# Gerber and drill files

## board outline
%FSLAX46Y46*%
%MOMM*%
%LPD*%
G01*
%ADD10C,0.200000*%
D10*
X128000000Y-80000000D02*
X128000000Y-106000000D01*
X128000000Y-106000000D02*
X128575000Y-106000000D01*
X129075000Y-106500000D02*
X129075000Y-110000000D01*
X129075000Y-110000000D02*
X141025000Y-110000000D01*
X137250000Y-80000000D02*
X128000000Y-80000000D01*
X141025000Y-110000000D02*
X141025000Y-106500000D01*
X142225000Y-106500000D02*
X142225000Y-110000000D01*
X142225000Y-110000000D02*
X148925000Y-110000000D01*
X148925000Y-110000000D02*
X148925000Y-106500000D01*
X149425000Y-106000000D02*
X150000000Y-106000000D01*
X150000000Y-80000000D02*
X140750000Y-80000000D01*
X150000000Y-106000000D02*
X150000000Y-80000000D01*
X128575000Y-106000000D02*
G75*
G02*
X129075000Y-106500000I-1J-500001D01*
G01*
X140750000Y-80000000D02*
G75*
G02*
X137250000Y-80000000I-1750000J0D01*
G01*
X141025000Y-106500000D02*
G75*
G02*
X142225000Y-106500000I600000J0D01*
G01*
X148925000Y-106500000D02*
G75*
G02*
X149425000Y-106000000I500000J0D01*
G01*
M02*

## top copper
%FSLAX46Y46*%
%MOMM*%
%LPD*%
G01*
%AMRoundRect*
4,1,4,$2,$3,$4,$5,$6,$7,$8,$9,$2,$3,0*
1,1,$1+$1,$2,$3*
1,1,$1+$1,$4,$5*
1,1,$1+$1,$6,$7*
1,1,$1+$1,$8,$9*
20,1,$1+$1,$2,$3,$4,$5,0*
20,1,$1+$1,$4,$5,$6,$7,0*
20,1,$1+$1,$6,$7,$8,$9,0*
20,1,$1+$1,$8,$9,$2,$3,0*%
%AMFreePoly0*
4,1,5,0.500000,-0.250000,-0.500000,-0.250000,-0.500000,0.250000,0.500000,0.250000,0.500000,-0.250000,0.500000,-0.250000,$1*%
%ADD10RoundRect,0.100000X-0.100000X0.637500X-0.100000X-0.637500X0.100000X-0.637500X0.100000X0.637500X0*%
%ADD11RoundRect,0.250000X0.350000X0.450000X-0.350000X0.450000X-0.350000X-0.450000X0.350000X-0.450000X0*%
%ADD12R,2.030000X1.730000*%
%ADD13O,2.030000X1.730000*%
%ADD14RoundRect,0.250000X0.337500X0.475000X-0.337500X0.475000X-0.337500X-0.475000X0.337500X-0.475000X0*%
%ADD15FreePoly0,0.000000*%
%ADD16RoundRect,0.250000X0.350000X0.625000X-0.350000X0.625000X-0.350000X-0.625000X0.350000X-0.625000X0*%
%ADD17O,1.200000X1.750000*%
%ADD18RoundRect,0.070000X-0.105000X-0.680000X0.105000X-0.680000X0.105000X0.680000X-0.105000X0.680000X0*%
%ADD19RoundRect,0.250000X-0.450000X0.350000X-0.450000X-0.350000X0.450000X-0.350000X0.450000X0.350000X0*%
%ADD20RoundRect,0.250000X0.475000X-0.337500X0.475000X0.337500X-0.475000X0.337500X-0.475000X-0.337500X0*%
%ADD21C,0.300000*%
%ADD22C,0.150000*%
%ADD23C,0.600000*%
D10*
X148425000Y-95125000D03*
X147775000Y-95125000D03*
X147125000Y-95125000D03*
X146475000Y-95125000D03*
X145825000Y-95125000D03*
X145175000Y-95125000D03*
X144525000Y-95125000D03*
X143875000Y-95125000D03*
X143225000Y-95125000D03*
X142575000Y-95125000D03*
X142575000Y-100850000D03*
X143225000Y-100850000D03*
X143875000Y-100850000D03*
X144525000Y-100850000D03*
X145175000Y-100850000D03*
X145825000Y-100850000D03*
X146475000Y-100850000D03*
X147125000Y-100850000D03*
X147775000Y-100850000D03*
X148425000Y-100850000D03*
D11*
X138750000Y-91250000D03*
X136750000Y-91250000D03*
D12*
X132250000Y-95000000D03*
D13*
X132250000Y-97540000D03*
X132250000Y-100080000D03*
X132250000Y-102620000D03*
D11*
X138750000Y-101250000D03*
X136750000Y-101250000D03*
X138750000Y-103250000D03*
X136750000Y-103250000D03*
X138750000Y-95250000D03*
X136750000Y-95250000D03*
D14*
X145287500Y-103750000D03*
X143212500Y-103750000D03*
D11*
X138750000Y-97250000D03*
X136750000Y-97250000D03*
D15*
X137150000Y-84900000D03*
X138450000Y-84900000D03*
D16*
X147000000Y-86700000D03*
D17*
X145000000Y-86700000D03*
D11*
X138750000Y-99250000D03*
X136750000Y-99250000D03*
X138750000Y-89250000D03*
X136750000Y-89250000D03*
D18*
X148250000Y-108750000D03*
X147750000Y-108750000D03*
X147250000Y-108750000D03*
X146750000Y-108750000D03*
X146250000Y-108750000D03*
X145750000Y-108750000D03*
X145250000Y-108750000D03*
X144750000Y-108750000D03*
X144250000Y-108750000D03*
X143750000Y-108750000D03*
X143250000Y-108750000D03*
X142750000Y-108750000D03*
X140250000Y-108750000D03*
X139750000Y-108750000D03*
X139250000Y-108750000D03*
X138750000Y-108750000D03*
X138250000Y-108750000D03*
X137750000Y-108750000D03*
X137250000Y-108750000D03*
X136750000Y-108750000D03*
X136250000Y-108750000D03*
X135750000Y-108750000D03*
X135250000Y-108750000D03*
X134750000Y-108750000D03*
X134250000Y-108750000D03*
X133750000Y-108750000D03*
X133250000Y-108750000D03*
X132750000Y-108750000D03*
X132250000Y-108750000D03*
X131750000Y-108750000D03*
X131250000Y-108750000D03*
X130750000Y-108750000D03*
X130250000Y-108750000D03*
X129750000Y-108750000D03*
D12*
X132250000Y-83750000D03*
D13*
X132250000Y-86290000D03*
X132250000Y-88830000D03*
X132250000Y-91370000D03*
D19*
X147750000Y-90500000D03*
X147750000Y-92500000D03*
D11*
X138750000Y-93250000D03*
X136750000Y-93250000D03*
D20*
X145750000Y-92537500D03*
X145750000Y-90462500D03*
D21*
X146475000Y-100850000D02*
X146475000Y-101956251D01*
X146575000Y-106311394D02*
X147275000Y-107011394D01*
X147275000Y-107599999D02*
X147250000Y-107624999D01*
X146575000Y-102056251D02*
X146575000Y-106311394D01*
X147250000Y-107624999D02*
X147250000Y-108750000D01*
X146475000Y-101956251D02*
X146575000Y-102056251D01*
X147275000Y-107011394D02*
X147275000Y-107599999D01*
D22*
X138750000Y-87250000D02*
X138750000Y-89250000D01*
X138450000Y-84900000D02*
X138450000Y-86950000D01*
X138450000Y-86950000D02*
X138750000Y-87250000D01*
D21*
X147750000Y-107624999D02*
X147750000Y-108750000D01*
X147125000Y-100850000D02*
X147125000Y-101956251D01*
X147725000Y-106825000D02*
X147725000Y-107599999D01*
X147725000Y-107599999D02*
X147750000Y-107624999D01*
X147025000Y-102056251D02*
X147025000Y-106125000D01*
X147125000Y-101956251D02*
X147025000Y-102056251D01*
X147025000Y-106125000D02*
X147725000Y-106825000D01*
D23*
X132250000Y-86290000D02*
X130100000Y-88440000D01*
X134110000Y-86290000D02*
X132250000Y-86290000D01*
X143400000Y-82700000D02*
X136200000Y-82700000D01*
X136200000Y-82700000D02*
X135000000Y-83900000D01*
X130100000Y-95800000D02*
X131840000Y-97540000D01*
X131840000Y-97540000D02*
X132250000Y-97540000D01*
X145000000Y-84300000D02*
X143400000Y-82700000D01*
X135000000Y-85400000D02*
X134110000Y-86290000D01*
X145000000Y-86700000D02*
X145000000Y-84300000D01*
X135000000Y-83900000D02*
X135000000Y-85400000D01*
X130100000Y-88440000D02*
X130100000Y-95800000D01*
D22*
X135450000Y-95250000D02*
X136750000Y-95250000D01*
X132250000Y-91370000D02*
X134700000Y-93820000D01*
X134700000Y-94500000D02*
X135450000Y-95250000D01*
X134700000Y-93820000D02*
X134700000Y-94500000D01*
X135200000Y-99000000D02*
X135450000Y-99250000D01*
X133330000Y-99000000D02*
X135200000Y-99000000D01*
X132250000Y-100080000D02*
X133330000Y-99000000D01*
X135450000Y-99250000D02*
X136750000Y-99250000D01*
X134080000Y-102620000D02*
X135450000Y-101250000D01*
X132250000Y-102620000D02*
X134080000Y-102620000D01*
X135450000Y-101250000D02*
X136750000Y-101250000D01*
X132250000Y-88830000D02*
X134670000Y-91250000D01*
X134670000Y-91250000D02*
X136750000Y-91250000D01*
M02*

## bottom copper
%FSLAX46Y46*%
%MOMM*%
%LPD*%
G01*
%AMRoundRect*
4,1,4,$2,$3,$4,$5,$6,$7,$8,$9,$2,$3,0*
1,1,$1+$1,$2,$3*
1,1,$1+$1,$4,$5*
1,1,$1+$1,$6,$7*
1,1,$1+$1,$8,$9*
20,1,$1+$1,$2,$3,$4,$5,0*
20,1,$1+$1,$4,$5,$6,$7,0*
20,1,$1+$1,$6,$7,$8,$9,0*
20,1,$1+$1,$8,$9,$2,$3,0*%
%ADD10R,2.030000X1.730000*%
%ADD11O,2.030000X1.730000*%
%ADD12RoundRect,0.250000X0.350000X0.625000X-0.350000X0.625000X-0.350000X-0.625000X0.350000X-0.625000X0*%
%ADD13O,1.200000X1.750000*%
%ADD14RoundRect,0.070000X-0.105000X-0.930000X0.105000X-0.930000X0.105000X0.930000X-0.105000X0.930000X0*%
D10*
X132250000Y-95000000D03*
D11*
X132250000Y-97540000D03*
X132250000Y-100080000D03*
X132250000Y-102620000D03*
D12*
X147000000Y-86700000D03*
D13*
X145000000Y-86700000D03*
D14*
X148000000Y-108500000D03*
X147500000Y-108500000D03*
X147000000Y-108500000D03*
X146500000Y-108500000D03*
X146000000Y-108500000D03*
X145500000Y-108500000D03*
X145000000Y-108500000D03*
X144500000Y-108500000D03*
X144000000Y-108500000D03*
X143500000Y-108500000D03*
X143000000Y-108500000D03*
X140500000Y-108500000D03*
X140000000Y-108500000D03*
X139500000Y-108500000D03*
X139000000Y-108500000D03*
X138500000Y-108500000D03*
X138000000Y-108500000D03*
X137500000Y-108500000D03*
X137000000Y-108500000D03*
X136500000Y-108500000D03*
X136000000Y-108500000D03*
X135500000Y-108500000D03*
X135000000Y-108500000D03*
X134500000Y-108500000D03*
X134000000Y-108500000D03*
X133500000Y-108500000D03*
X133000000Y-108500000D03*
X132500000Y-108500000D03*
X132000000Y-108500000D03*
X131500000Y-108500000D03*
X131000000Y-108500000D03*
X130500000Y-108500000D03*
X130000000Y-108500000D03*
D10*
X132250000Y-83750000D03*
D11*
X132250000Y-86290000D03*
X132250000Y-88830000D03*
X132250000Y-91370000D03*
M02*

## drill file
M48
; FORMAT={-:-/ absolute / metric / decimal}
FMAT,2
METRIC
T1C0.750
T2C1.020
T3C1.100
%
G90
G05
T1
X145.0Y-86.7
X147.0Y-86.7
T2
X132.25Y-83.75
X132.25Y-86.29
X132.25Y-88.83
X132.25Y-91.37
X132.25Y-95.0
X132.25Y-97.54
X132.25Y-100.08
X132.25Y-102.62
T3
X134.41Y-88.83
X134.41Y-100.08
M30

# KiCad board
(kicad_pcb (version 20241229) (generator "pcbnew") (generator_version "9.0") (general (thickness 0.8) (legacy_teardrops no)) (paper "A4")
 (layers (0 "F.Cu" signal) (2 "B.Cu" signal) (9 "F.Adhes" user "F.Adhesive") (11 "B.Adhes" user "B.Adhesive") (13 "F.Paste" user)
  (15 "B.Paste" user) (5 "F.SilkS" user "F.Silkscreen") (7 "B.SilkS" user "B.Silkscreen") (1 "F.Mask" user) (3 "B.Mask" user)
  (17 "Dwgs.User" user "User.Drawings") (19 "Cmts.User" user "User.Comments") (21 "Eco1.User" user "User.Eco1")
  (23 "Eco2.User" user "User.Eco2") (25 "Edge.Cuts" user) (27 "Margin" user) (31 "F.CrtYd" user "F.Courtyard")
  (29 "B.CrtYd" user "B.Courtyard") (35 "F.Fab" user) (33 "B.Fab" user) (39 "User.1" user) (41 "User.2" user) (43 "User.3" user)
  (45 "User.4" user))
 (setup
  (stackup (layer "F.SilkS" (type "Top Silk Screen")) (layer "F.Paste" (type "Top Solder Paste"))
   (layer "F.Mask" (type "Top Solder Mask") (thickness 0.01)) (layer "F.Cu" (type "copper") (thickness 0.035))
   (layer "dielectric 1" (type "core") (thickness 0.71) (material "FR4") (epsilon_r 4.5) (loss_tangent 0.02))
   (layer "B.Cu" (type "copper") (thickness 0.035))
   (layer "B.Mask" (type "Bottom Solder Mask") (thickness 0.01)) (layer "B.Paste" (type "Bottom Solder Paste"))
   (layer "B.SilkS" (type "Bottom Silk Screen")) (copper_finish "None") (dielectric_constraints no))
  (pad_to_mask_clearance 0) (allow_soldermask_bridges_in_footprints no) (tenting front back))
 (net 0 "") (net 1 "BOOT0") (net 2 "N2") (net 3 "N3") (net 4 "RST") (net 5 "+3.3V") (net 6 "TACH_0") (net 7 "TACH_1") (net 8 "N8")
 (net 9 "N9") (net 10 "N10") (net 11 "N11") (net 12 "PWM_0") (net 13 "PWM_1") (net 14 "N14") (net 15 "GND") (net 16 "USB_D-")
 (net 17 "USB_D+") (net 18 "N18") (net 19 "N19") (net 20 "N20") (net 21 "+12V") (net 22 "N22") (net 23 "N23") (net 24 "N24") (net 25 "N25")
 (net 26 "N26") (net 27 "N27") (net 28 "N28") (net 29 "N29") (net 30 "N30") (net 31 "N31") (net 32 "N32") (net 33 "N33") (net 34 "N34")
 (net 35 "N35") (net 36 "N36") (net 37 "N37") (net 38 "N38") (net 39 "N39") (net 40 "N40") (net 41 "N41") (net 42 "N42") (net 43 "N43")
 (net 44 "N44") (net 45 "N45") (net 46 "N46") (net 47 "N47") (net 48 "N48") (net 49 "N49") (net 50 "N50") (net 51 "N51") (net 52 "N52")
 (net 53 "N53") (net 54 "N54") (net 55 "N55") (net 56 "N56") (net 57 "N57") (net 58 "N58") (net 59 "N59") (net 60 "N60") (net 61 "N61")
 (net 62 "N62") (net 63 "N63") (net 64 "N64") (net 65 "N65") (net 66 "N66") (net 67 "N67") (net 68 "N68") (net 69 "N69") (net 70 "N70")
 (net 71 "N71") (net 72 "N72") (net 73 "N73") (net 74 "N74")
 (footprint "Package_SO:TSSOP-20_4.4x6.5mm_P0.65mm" (layer "F.Cu") (at 145.5 97.9875 -90)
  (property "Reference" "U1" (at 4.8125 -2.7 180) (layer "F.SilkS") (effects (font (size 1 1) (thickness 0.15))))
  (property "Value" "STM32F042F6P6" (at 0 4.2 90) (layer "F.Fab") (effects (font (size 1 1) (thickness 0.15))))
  (pad "1" smd roundrect (at -2.8625 -2.925 270) (size 1.475 0.4) (layers "F.Cu" "F.Mask" "F.Paste") (roundrect_rratio 0.25) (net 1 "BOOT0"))
  (pad "2" smd roundrect (at -2.8625 -2.275 270) (size 1.475 0.4) (layers "F.Cu" "F.Mask" "F.Paste") (roundrect_rratio 0.25) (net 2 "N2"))
  (pad "3" smd roundrect (at -2.8625 -1.625 270) (size 1.475 0.4) (layers "F.Cu" "F.Mask" "F.Paste") (roundrect_rratio 0.25) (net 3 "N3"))
  (pad "4" smd roundrect (at -2.8625 -0.975 270) (size 1.475 0.4) (layers "F.Cu" "F.Mask" "F.Paste") (roundrect_rratio 0.25) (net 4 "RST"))
  (pad "5" smd roundrect (at -2.8625 -0.325 270) (size 1.475 0.4) (layers "F.Cu" "F.Mask" "F.Paste") (roundrect_rratio 0.25) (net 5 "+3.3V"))
  (pad "6" smd roundrect (at -2.8625 0.325 270) (size 1.475 0.4) (layers "F.Cu" "F.Mask" "F.Paste") (roundrect_rratio 0.25) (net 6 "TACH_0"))
  (pad "7" smd roundrect (at -2.8625 0.975 270) (size 1.475 0.4) (layers "F.Cu" "F.Mask" "F.Paste") (roundrect_rratio 0.25) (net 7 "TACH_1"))
  (pad "8" smd roundrect (at -2.8625 1.625 270) (size 1.475 0.4) (layers "F.Cu" "F.Mask" "F.Paste") (roundrect_rratio 0.25) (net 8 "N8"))
  (pad "9" smd roundrect (at -2.8625 2.275 270) (size 1.475 0.4) (layers "F.Cu" "F.Mask" "F.Paste") (roundrect_rratio 0.25) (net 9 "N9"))
  (pad "10" smd roundrect (at -2.8625 2.925 270) (size 1.475 0.4) (layers "F.Cu" "F.Mask" "F.Paste") (roundrect_rratio 0.25) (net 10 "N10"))
  (pad "11" smd roundrect (at 2.8625 2.925 270) (size 1.475 0.4) (layers "F.Cu" "F.Mask" "F.Paste") (roundrect_rratio 0.25) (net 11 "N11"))
  (pad "12" smd roundrect (at 2.8625 2.275 270) (size 1.475 0.4) (layers "F.Cu" "F.Mask" "F.Paste") (roundrect_rratio 0.25) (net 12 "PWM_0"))
  (pad "13" smd roundrect (at 2.8625 1.625 270) (size 1.475 0.4) (layers "F.Cu" "F.Mask" "F.Paste") (roundrect_rratio 0.25) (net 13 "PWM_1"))
  (pad "14" smd roundrect (at 2.8625 0.975 270) (size 1.475 0.4) (layers "F.Cu" "F.Mask" "F.Paste") (roundrect_rratio 0.25) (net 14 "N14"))
  (pad "15" smd roundrect (at 2.8625 0.325 270) (size 1.475 0.4) (layers "F.Cu" "F.Mask" "F.Paste") (roundrect_rratio 0.25) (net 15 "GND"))
  (pad "16" smd roundrect (at 2.8625 -0.325 270) (size 1.475 0.4) (layers "F.Cu" "F.Mask" "F.Paste") (roundrect_rratio 0.25) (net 5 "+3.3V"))
  (pad "17" smd roundrect (at 2.8625 -0.975 270) (size 1.475 0.4) (layers "F.Cu" "F.Mask" "F.Paste") (roundrect_rratio 0.25)
   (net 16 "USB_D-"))
  (pad "18" smd roundrect (at 2.8625 -1.625 270) (size 1.475 0.4) (layers "F.Cu" "F.Mask" "F.Paste") (roundrect_rratio 0.25)
   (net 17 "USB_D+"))
  (pad "19" smd roundrect (at 2.8625 -2.275 270) (size 1.475 0.4) (layers "F.Cu" "F.Mask" "F.Paste") (roundrect_rratio 0.25) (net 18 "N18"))
  (pad "20" smd roundrect (at 2.8625 -2.925 270) (size 1.475 0.4) (layers "F.Cu" "F.Mask" "F.Paste") (roundrect_rratio 0.25) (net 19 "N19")))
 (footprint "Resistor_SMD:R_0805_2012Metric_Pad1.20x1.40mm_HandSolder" (layer "F.Cu") (at 137.75 91.25 180)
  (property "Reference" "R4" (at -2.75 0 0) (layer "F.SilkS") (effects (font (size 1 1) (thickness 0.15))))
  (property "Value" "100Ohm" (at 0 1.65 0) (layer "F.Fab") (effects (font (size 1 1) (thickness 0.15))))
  (pad "1" smd roundrect (at -1 0 180) (size 1.2 1.4) (layers "F.Cu" "F.Mask" "F.Paste") (roundrect_rratio 0.208333) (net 6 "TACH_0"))
  (pad "2" smd roundrect (at 1 0 180) (size 1.2 1.4) (layers "F.Cu" "F.Mask" "F.Paste") (roundrect_rratio 0.208333) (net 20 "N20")))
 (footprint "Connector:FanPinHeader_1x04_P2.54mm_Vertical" (layer "F.Cu") (at 132.25 95 -90)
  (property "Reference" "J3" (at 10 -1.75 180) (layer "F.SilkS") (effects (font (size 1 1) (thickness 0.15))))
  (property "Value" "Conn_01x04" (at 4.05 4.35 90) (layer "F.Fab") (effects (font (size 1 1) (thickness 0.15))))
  (pad "" np_thru_hole circle (at 5.08 -2.16) (size 1.1 1.1) (drill 1.1) (layers "*.Cu" "*.Mask"))
  (pad "1" thru_hole rect (at 0 0) (size 2.03 1.73) (drill 1.02) (layers "*.Cu" "*.Mask") (remove_unused_layers no) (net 15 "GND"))
  (pad "2" thru_hole oval (at 2.54 0) (size 2.03 1.73) (drill 1.02) (layers "*.Cu" "*.Mask") (remove_unused_layers no) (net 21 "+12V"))
  (pad "3" thru_hole oval (at 5.08 0) (size 2.03 1.73) (drill 1.02) (layers "*.Cu" "*.Mask") (remove_unused_layers no) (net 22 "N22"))
  (pad "4" thru_hole oval (at 7.62 0) (size 2.03 1.73) (drill 1.02) (layers "*.Cu" "*.Mask") (remove_unused_layers no) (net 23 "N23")))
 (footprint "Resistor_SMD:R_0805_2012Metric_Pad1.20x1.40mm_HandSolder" (layer "F.Cu") (at 137.75 101.25 180)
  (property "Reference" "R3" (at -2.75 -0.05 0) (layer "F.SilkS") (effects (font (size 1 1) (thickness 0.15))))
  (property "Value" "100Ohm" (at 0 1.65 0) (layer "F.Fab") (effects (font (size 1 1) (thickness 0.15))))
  (pad "1" smd roundrect (at -1 0 180) (size 1.2 1.4) (layers "F.Cu" "F.Mask" "F.Paste") (roundrect_rratio 0.208333) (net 13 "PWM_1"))
  (pad "2" smd roundrect (at 1 0 180) (size 1.2 1.4) (layers "F.Cu" "F.Mask" "F.Paste") (roundrect_rratio 0.208333) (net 23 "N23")))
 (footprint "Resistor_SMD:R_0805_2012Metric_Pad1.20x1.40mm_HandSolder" (layer "F.Cu") (at 137.75 103.25 180)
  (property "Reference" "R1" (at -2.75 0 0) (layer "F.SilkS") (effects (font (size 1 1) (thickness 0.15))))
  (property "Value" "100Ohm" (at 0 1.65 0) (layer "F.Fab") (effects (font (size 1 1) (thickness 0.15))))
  (pad "1" smd roundrect (at -1 0 180) (size 1.2 1.4) (layers "F.Cu" "F.Mask" "F.Paste") (roundrect_rratio 0.208333) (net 4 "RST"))
  (pad "2" smd roundrect (at 1 0 180) (size 1.2 1.4) (layers "F.Cu" "F.Mask" "F.Paste") (roundrect_rratio 0.208333) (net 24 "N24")))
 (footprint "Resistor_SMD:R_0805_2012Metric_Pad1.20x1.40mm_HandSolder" (layer "F.Cu") (at 137.75 95.25 180)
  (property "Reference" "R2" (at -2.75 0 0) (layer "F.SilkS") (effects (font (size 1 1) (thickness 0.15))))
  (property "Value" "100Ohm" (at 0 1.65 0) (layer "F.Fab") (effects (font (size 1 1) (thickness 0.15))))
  (pad "1" smd roundrect (at -1 0 180) (size 1.2 1.4) (layers "F.Cu" "F.Mask" "F.Paste") (roundrect_rratio 0.208333) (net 12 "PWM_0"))
  (pad "2" smd roundrect (at 1 0 180) (size 1.2 1.4) (layers "F.Cu" "F.Mask" "F.Paste") (roundrect_rratio 0.208333) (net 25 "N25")))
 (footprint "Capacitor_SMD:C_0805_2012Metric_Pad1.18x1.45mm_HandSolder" (layer "F.Cu") (at 144.25 103.75 180)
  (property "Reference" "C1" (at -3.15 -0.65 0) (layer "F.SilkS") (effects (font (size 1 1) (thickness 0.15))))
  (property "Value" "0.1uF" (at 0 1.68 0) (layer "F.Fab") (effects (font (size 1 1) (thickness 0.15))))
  (pad "1" smd roundrect (at -1.0375 0 180) (size 1.175 1.45) (layers "F.Cu" "F.Mask" "F.Paste") (roundrect_rratio 0.212766) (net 5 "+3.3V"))
  (pad "2" smd roundrect (at 1.0375 0 180) (size 1.175 1.45) (layers "F.Cu" "F.Mask" "F.Paste") (roundrect_rratio 0.212766) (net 15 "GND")))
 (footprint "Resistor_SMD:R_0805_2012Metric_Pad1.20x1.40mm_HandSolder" (layer "F.Cu") (at 137.75 97.25 180)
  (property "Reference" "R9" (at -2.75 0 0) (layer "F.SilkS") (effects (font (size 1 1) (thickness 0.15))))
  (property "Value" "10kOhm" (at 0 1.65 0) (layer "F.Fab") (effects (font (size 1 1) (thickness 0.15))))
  (pad "1" smd roundrect (at -1 0 180) (size 1.2 1.4) (layers "F.Cu" "F.Mask" "F.Paste") (roundrect_rratio 0.208333) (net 5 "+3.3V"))
  (pad "2" smd roundrect (at 1 0 180) (size 1.2 1.4) (layers "F.Cu" "F.Mask" "F.Paste") (roundrect_rratio 0.208333) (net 7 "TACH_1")))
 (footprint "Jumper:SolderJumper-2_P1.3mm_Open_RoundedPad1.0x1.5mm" (layer "F.Cu") (at 137.8 84.9)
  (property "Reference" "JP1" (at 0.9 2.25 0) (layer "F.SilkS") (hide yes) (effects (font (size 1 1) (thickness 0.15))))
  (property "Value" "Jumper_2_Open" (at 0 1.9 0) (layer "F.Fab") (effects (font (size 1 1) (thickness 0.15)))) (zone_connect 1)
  (pad "1" smd custom (at -0.65 0) (size 1 0.5) (layers "F.Cu" "F.Mask") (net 5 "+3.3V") (zone_connect 2) (thermal_bridge_angle 45)
   (options (clearance outline) (anchor rect)) (primitives))
  (pad "2" smd custom (at 0.65 0) (size 1 0.5) (layers "F.Cu" "F.Mask") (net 1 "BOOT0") (zone_connect 2) (thermal_bridge_angle 45)
   (options (clearance outline) (anchor rect)) (primitives)))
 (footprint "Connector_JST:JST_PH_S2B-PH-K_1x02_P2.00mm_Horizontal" (layer "F.Cu") (at 147 86.7 180)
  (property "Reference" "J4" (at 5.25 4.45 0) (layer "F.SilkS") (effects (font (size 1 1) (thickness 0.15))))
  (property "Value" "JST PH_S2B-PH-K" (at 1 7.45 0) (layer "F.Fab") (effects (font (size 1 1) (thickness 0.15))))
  (pad "1" thru_hole roundrect (at 0 0 180) (size 1.2 1.75) (drill 0.75) (layers "*.Cu" "*.Mask") (remove_unused_layers no)
   (roundrect_rratio 0.208333) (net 15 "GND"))
  (pad "2" thru_hole oval (at 2 0 180) (size 1.2 1.75) (drill 0.75) (layers "*.Cu" "*.Mask") (remove_unused_layers no) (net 21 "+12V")))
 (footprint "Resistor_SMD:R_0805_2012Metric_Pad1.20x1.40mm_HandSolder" (layer "F.Cu") (at 137.75 99.25 180)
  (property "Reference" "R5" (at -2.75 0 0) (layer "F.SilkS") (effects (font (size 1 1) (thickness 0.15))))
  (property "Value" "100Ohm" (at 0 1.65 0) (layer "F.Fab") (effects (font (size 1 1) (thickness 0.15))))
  (pad "1" smd roundrect (at -1 0 180) (size 1.2 1.4) (layers "F.Cu" "F.Mask" "F.Paste") (roundrect_rratio 0.208333) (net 7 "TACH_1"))
  (pad "2" smd roundrect (at 1 0 180) (size 1.2 1.4) (layers "F.Cu" "F.Mask" "F.Paste") (roundrect_rratio 0.208333) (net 22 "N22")))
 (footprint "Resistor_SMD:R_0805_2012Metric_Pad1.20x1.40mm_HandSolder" (layer "F.Cu") (at 137.75 89.25 180)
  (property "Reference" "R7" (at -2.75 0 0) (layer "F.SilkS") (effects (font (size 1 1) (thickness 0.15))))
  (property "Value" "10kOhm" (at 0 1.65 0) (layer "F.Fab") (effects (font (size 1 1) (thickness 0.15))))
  (pad "1" smd roundrect (at -1 0 180) (size 1.2 1.4) (layers "F.Cu" "F.Mask" "F.Paste") (roundrect_rratio 0.208333) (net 1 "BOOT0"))
  (pad "2" smd roundrect (at 1 0 180) (size 1.2 1.4) (layers "F.Cu" "F.Mask" "F.Paste") (roundrect_rratio 0.208333) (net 15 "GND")))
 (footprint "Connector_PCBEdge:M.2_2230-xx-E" (layer "F.Cu") (at 139 106)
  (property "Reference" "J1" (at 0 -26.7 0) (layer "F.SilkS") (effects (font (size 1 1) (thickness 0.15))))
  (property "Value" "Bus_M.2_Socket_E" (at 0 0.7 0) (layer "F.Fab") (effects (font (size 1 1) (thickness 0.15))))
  (fp_line (start -11 -26) (end -11 0) (stroke (width 0.2) (type solid)) (layer "Edge.Cuts"))
  (fp_line (start -11 0) (end -10.425 0) (stroke (width 0.2) (type solid)) (layer "Edge.Cuts"))
  (fp_line (start -9.925 0.5) (end -9.925 4) (stroke (width 0.2) (type solid)) (layer "Edge.Cuts"))
  (fp_line (start -9.925 4) (end 2.025 4) (stroke (width 0.2) (type solid)) (layer "Edge.Cuts"))
  (fp_line (start -1.75 -26) (end -11 -26) (stroke (width 0.2) (type solid)) (layer "Edge.Cuts"))
  (fp_line (start 2.025 4) (end 2.025 0.5) (stroke (width 0.2) (type solid)) (layer "Edge.Cuts"))
  (fp_line (start 3.225 0.5) (end 3.225 4) (stroke (width 0.2) (type solid)) (layer "Edge.Cuts"))
  (fp_line (start 3.225 4) (end 9.925 4) (stroke (width 0.2) (type solid)) (layer "Edge.Cuts"))
  (fp_line (start 9.925 4) (end 9.925 0.5) (stroke (width 0.2) (type solid)) (layer "Edge.Cuts"))
  (fp_line (start 10.425 0) (end 11 0) (stroke (width 0.2) (type solid)) (layer "Edge.Cuts"))
  (fp_line (start 11 -26) (end 1.75 -26) (stroke (width 0.2) (type solid)) (layer "Edge.Cuts"))
  (fp_line (start 11 0) (end 11 -26) (stroke (width 0.2) (type solid)) (layer "Edge.Cuts"))
  (fp_arc (start -10.425 0) (mid -10.071447 0.146447) (end -9.925 0.5) (stroke (width 0.2) (type solid)) (layer "Edge.Cuts"))
  (fp_arc (start 1.75 -26) (mid 0 -24.25) (end -1.75 -26) (stroke (width 0.2) (type solid)) (layer "Edge.Cuts"))
  (fp_arc (start 2.025 0.5) (mid 2.625 -0.1) (end 3.225 0.5) (stroke (width 0.2) (type solid)) (layer "Edge.Cuts"))
  (fp_arc (start 9.925 0.5) (mid 10.071447 0.146447) (end 10.425 0) (stroke (width 0.2) (type solid)) (layer "Edge.Cuts"))
  (pad "1" connect roundrect (at 9.25 2.75) (size 0.35 1.5) (layers "F.Cu" "F.Mask") (roundrect_rratio 0.2) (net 15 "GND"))
  (pad "2" connect roundrect (at 9 2.5) (size 0.35 2) (layers "B.Cu" "B.Mask") (roundrect_rratio 0.2) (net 5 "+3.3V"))
  (pad "3" connect roundrect (at 8.75 2.75) (size 0.35 1.5) (layers "F.Cu" "F.Mask") (roundrect_rratio 0.2) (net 17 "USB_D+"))
  (pad "4" connect roundrect (at 8.5 2.5) (size 0.35 2) (layers "B.Cu" "B.Mask") (roundrect_rratio 0.2) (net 5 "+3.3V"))
  (pad "5" connect roundrect (at 8.25 2.75) (size 0.35 1.5) (layers "F.Cu" "F.Mask") (roundrect_rratio 0.2) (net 16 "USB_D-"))
  (pad "6" connect roundrect (at 8 2.5) (size 0.35 2) (layers "B.Cu" "B.Mask") (roundrect_rratio 0.2) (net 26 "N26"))
  (pad "7" connect roundrect (at 7.75 2.75) (size 0.35 1.5) (layers "F.Cu" "F.Mask") (roundrect_rratio 0.2) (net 15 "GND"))
  (pad "8" connect roundrect (at 7.5 2.5) (size 0.35 2) (layers "B.Cu" "B.Mask") (roundrect_rratio 0.2) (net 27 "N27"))
  (pad "9" connect roundrect (at 7.25 2.75) (size 0.35 1.5) (layers "F.Cu" "F.Mask") (roundrect_rratio 0.2) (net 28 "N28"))
  (pad "10" connect roundrect (at 7 2.5) (size 0.35 2) (layers "B.Cu" "B.Mask") (roundrect_rratio 0.2) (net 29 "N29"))
  (pad "11" connect roundrect (at 6.75 2.75) (size 0.35 1.5) (layers "F.Cu" "F.Mask") (roundrect_rratio 0.2) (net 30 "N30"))
  (pad "12" connect roundrect (at 6.5 2.5) (size 0.35 2) (layers "B.Cu" "B.Mask") (roundrect_rratio 0.2) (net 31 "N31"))
  (pad "13" connect roundrect (at 6.25 2.75) (size 0.35 1.5) (layers "F.Cu" "F.Mask") (roundrect_rratio 0.2) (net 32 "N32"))
  (pad "14" connect roundrect (at 6 2.5) (size 0.35 2) (layers "B.Cu" "B.Mask") (roundrect_rratio 0.2) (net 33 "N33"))
  (pad "15" connect roundrect (at 5.75 2.75) (size 0.35 1.5) (layers "F.Cu" "F.Mask") (roundrect_rratio 0.2) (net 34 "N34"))
  (pad "16" connect roundrect (at 5.5 2.5) (size 0.35 2) (layers "B.Cu" "B.Mask") (roundrect_rratio 0.2) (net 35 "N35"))
  (pad "17" connect roundrect (at 5.25 2.75) (size 0.35 1.5) (layers "F.Cu" "F.Mask") (roundrect_rratio 0.2) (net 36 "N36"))
  (pad "18" connect roundrect (at 5 2.5) (size 0.35 2) (layers "B.Cu" "B.Mask") (roundrect_rratio 0.2) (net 15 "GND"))
  (pad "19" connect roundrect (at 4.75 2.75) (size 0.35 1.5) (layers "F.Cu" "F.Mask") (roundrect_rratio 0.2) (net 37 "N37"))
  (pad "20" connect roundrect (at 4.5 2.5) (size 0.35 2) (layers "B.Cu" "B.Mask") (roundrect_rratio 0.2) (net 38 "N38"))
  (pad "21" connect roundrect (at 4.25 2.75) (size 0.35 1.5) (layers "F.Cu" "F.Mask") (roundrect_rratio 0.2) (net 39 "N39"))
  (pad "22" connect roundrect (at 4 2.5) (size 0.35 2) (layers "B.Cu" "B.Mask") (roundrect_rratio 0.2) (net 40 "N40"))
  (pad "23" connect roundrect (at 3.75 2.75) (size 0.35 1.5) (layers "F.Cu" "F.Mask") (roundrect_rratio 0.2) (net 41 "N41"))
  (pad "32" connect roundrect (at 1.5 2.5) (size 0.35 2) (layers "B.Cu" "B.Mask") (roundrect_rratio 0.2) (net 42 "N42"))
  (pad "33" connect roundrect (at 1.25 2.75) (size 0.35 1.5) (layers "F.Cu" "F.Mask") (roundrect_rratio 0.2) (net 15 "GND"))
  (pad "34" connect roundrect (at 1 2.5) (size 0.35 2) (layers "B.Cu" "B.Mask") (roundrect_rratio 0.2) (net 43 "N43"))
  (pad "35" connect roundrect (at 0.75 2.75) (size 0.35 1.5) (layers "F.Cu" "F.Mask") (roundrect_rratio 0.2) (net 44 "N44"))
  (pad "36" connect roundrect (at 0.5 2.5) (size 0.35 2) (layers "B.Cu" "B.Mask") (roundrect_rratio 0.2) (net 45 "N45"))
  (pad "37" connect roundrect (at 0.25 2.75) (size 0.35 1.5) (layers "F.Cu" "F.Mask") (roundrect_rratio 0.2) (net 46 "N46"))
  (pad "38" connect roundrect (at 0 2.5) (size 0.35 2) (layers "B.Cu" "B.Mask") (roundrect_rratio 0.2) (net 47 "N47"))
  (pad "39" connect roundrect (at -0.25 2.75) (size 0.35 1.5) (layers "F.Cu" "F.Mask") (roundrect_rratio 0.2) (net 15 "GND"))
  (pad "40" connect roundrect (at -0.5 2.5) (size 0.35 2) (layers "B.Cu" "B.Mask") (roundrect_rratio 0.2) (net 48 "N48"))
  (pad "41" connect roundrect (at -0.75 2.75) (size 0.35 1.5) (layers "F.Cu" "F.Mask") (roundrect_rratio 0.2) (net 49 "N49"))
  (pad "42" connect roundrect (at -1 2.5) (size 0.35 2) (layers "B.Cu" "B.Mask") (roundrect_rratio 0.2) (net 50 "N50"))
  (pad "43" connect roundrect (at -1.25 2.75) (size 0.35 1.5) (layers "F.Cu" "F.Mask") (roundrect_rratio 0.2) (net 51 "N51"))
  (pad "44" connect roundrect (at -1.5 2.5) (size 0.35 2) (layers "B.Cu" "B.Mask") (roundrect_rratio 0.2) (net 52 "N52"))
  (pad "45" connect roundrect (at -1.75 2.75) (size 0.35 1.5) (layers "F.Cu" "F.Mask") (roundrect_rratio 0.2) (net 15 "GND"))
  (pad "46" connect roundrect (at -2 2.5) (size 0.35 2) (layers "B.Cu" "B.Mask") (roundrect_rratio 0.2) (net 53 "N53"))
  (pad "47" connect roundrect (at -2.25 2.75) (size 0.35 1.5) (layers "F.Cu" "F.Mask") (roundrect_rratio 0.2) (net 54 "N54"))
  (pad "48" connect roundrect (at -2.5 2.5) (size 0.35 2) (layers "B.Cu" "B.Mask") (roundrect_rratio 0.2) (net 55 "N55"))
  (pad "49" connect roundrect (at -2.75 2.75) (size 0.35 1.5) (layers "F.Cu" "F.Mask") (roundrect_rratio 0.2) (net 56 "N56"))
  (pad "50" connect roundrect (at -3 2.5) (size 0.35 2) (layers "B.Cu" "B.Mask") (roundrect_rratio 0.2) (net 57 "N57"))
  (pad "51" connect roundrect (at -3.25 2.75) (size 0.35 1.5) (layers "F.Cu" "F.Mask") (roundrect_rratio 0.2) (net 15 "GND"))
  (pad "52" connect roundrect (at -3.5 2.5) (size 0.35 2) (layers "B.Cu" "B.Mask") (roundrect_rratio 0.2) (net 24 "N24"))
  (pad "53" connect roundrect (at -3.75 2.75) (size 0.35 1.5) (layers "F.Cu" "F.Mask") (roundrect_rratio 0.2) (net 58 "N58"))
  (pad "54" connect roundrect (at -4 2.5) (size 0.35 2) (layers "B.Cu" "B.Mask") (roundrect_rratio 0.2) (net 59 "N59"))
  (pad "55" connect roundrect (at -4.25 2.75) (size 0.35 1.5) (layers "F.Cu" "F.Mask") (roundrect_rratio 0.2) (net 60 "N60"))
  (pad "56" connect roundrect (at -4.5 2.5) (size 0.35 2) (layers "B.Cu" "B.Mask") (roundrect_rratio 0.2) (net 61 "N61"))
  (pad "57" connect roundrect (at -4.75 2.75) (size 0.35 1.5) (layers "F.Cu" "F.Mask") (roundrect_rratio 0.2) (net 15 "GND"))
  (pad "58" connect roundrect (at -5 2.5) (size 0.35 2) (layers "B.Cu" "B.Mask") (roundrect_rratio 0.2) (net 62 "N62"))
  (pad "59" connect roundrect (at -5.25 2.75) (size 0.35 1.5) (layers "F.Cu" "F.Mask") (roundrect_rratio 0.2) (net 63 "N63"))
  (pad "60" connect roundrect (at -5.5 2.5) (size 0.35 2) (layers "B.Cu" "B.Mask") (roundrect_rratio 0.2) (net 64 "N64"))
  (pad "61" connect roundrect (at -5.75 2.75) (size 0.35 1.5) (layers "F.Cu" "F.Mask") (roundrect_rratio 0.2) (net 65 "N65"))
  (pad "62" connect roundrect (at -6 2.5) (size 0.35 2) (layers "B.Cu" "B.Mask") (roundrect_rratio 0.2) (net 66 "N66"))
  (pad "63" connect roundrect (at -6.25 2.75) (size 0.35 1.5) (layers "F.Cu" "F.Mask") (roundrect_rratio 0.2) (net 15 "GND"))
  (pad "64" connect roundrect (at -6.5 2.5) (size 0.35 2) (layers "B.Cu" "B.Mask") (roundrect_rratio 0.2) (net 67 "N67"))
  (pad "65" connect roundrect (at -6.75 2.75) (size 0.35 1.5) (layers "F.Cu" "F.Mask") (roundrect_rratio 0.2) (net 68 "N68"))
  (pad "66" connect roundrect (at -7 2.5) (size 0.35 2) (layers "B.Cu" "B.Mask") (roundrect_rratio 0.2) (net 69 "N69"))
  (pad "67" connect roundrect (at -7.25 2.75) (size 0.35 1.5) (layers "F.Cu" "F.Mask") (roundrect_rratio 0.2) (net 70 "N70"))
  (pad "68" connect roundrect (at -7.5 2.5) (size 0.35 2) (layers "B.Cu" "B.Mask") (roundrect_rratio 0.2) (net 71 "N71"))
  (pad "69" connect roundrect (at -7.75 2.75) (size 0.35 1.5) (layers "F.Cu" "F.Mask") (roundrect_rratio 0.2) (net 15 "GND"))
  (pad "70" connect roundrect (at -8 2.5) (size 0.35 2) (layers "B.Cu" "B.Mask") (roundrect_rratio 0.2) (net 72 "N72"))
  (pad "71" connect roundrect (at -8.25 2.75) (size 0.35 1.5) (layers "F.Cu" "F.Mask") (roundrect_rratio 0.2) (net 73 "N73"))
  (pad "72" connect roundrect (at -8.5 2.5) (size 0.35 2) (layers "B.Cu" "B.Mask") (roundrect_rratio 0.2) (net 5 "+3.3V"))
  (pad "73" connect roundrect (at -8.75 2.75) (size 0.35 1.5) (layers "F.Cu" "F.Mask") (roundrect_rratio 0.2) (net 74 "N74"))
  (pad "74" connect roundrect (at -9 2.5) (size 0.35 2) (layers "B.Cu" "B.Mask") (roundrect_rratio 0.2) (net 5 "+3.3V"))
  (pad "75" connect roundrect (at -9.25 2.75) (size 0.35 1.5) (layers "F.Cu" "F.Mask") (roundrect_rratio 0.2) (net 15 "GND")))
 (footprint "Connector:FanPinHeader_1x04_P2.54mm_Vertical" (layer "F.Cu") (at 132.25 83.75 -90)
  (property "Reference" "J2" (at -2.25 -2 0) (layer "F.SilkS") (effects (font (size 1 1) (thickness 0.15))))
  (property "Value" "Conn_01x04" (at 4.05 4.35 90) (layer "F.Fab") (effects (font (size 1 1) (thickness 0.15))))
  (pad "" np_thru_hole circle (at 5.08 -2.16) (size 1.1 1.1) (drill 1.1) (layers "*.Cu" "*.Mask"))
  (pad "1" thru_hole rect (at 0 0) (size 2.03 1.73) (drill 1.02) (layers "*.Cu" "*.Mask") (remove_unused_layers no) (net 15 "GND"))
  (pad "2" thru_hole oval (at 2.54 0) (size 2.03 1.73) (drill 1.02) (layers "*.Cu" "*.Mask") (remove_unused_layers no) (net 21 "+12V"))
  (pad "3" thru_hole oval (at 5.08 0) (size 2.03 1.73) (drill 1.02) (layers "*.Cu" "*.Mask") (remove_unused_layers no) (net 20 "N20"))
  (pad "4" thru_hole oval (at 7.62 0) (size 2.03 1.73) (drill 1.02) (layers "*.Cu" "*.Mask") (remove_unused_layers no) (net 25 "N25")))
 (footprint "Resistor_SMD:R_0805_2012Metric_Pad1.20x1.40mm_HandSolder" (layer "F.Cu") (at 147.75 91.5 -90)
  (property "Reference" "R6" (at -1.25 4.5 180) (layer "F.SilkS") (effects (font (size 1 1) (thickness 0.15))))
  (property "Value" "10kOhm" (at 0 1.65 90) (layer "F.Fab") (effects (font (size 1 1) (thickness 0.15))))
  (pad "1" smd roundrect (at -1 0 270) (size 1.2 1.4) (layers "F.Cu" "F.Mask" "F.Paste") (roundrect_rratio 0.208333) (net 5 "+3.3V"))
  (pad "2" smd roundrect (at 1 0 270) (size 1.2 1.4) (layers "F.Cu" "F.Mask" "F.Paste") (roundrect_rratio 0.208333) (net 4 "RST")))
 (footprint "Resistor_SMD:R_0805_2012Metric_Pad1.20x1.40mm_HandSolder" (layer "F.Cu") (at 137.75 93.25 180)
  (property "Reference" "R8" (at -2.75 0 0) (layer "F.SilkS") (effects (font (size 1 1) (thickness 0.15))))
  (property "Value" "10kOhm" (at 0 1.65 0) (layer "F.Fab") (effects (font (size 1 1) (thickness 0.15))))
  (pad "1" smd roundrect (at -1 0 180) (size 1.2 1.4) (layers "F.Cu" "F.Mask" "F.Paste") (roundrect_rratio 0.208333) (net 5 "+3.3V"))
  (pad "2" smd roundrect (at 1 0 180) (size 1.2 1.4) (layers "F.Cu" "F.Mask" "F.Paste") (roundrect_rratio 0.208333) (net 6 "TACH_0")))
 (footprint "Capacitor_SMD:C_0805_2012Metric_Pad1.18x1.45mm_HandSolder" (layer "F.Cu") (at 145.75 91.5 90)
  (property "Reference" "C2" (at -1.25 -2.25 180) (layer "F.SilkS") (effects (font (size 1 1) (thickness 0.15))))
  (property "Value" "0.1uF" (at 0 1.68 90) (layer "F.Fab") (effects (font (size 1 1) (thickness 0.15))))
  (pad "1" smd roundrect (at -1.0375 0 90) (size 1.175 1.45) (layers "F.Cu" "F.Mask" "F.Paste") (roundrect_rratio 0.212766) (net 5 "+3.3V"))
  (pad "2" smd roundrect (at 1.0375 0 90) (size 1.175 1.45) (layers "F.Cu" "F.Mask" "F.Paste") (roundrect_rratio 0.212766) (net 15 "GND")))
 (segment (start 146.475 100.85) (end 146.475 101.956251) (width 0.3) (layer "F.Cu") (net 16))
 (segment (start 146.575 106.311394) (end 147.275 107.011394) (width 0.3) (layer "F.Cu") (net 16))
 (segment (start 147.275 107.599999) (end 147.25 107.624999) (width 0.3) (layer "F.Cu") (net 16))
 (segment (start 146.575 102.056251) (end 146.575 106.311394) (width 0.3) (layer "F.Cu") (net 16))
 (segment (start 147.25 107.624999) (end 147.25 108.75) (width 0.3) (layer "F.Cu") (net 16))
 (segment (start 146.475 101.956251) (end 146.575 102.056251) (width 0.3) (layer "F.Cu") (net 16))
 (segment (start 147.275 107.011394) (end 147.275 107.599999) (width 0.3) (layer "F.Cu") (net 16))
 (segment (start 138.75 87.25) (end 138.75 89.25) (width 0.15) (layer "F.Cu") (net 1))
 (segment (start 138.45 84.9) (end 138.45 86.95) (width 0.15) (layer "F.Cu") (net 1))
 (segment (start 138.45 86.95) (end 138.75 87.25) (width 0.15) (layer "F.Cu") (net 1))
 (segment (start 147.75 107.624999) (end 147.75 108.75) (width 0.3) (layer "F.Cu") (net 17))
 (segment (start 147.125 100.85) (end 147.125 101.956251) (width 0.3) (layer "F.Cu") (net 17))
 (segment (start 147.725 106.825) (end 147.725 107.599999) (width 0.3) (layer "F.Cu") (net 17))
 (segment (start 147.725 107.599999) (end 147.75 107.624999) (width 0.3) (layer "F.Cu") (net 17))
 (segment (start 147.025 102.056251) (end 147.025 106.125) (width 0.3) (layer "F.Cu") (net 17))
 (segment (start 147.125 101.956251) (end 147.025 102.056251) (width 0.3) (layer "F.Cu") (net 17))
 (segment (start 147.025 106.125) (end 147.725 106.825) (width 0.3) (layer "F.Cu") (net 17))
 (segment (start 132.25 86.29) (end 130.1 88.44) (width 0.6) (layer "F.Cu") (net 21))
 (segment (start 134.11 86.29) (end 132.25 86.29) (width 0.6) (layer "F.Cu") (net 21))
 (segment (start 143.4 82.7) (end 136.2 82.7) (width 0.6) (layer "F.Cu") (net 21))
 (segment (start 136.2 82.7) (end 135 83.9) (width 0.6) (layer "F.Cu") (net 21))
 (segment (start 130.1 95.8) (end 131.84 97.54) (width 0.6) (layer "F.Cu") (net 21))
 (segment (start 131.84 97.54) (end 132.25 97.54) (width 0.6) (layer "F.Cu") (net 21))
 (segment (start 145 84.3) (end 143.4 82.7) (width 0.6) (layer "F.Cu") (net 21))
 (segment (start 135 85.4) (end 134.11 86.29) (width 0.6) (layer "F.Cu") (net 21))
 (segment (start 145 86.7) (end 145 84.3) (width 0.6) (layer "F.Cu") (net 21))
 (segment (start 135 83.9) (end 135 85.4) (width 0.6) (layer "F.Cu") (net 21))
 (segment (start 130.1 88.44) (end 130.1 95.8) (width 0.6) (layer "F.Cu") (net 21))
 (segment (start 135.45 95.25) (end 136.75 95.25) (width 0.15) (layer "F.Cu") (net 25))
 (segment (start 132.25 91.37) (end 134.7 93.82) (width 0.15) (layer "F.Cu") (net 25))
 (segment (start 134.7 94.5) (end 135.45 95.25) (width 0.15) (layer "F.Cu") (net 25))
 (segment (start 134.7 93.82) (end 134.7 94.5) (width 0.15) (layer "F.Cu") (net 25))
 (segment (start 135.2 99) (end 135.45 99.25) (width 0.15) (layer "F.Cu") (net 22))
 (segment (start 133.33 99) (end 135.2 99) (width 0.15) (layer "F.Cu") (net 22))
 (segment (start 132.25 100.08) (end 133.33 99) (width 0.15) (layer "F.Cu") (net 22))
 (segment (start 135.45 99.25) (end 136.75 99.25) (width 0.15) (layer "F.Cu") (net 22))
 (segment (start 134.08 102.62) (end 135.45 101.25) (width 0.15) (layer "F.Cu") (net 23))
 (segment (start 132.25 102.62) (end 134.08 102.62) (width 0.15) (layer "F.Cu") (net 23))
 (segment (start 135.45 101.25) (end 136.75 101.25) (width 0.15) (layer "F.Cu") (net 23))
 (segment (start 132.25 88.83) (end 134.67 91.25) (width 0.15) (layer "F.Cu") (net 20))
 (segment (start 134.67 91.25) (end 136.75 91.25) (width 0.15) (layer "F.Cu") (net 20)))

